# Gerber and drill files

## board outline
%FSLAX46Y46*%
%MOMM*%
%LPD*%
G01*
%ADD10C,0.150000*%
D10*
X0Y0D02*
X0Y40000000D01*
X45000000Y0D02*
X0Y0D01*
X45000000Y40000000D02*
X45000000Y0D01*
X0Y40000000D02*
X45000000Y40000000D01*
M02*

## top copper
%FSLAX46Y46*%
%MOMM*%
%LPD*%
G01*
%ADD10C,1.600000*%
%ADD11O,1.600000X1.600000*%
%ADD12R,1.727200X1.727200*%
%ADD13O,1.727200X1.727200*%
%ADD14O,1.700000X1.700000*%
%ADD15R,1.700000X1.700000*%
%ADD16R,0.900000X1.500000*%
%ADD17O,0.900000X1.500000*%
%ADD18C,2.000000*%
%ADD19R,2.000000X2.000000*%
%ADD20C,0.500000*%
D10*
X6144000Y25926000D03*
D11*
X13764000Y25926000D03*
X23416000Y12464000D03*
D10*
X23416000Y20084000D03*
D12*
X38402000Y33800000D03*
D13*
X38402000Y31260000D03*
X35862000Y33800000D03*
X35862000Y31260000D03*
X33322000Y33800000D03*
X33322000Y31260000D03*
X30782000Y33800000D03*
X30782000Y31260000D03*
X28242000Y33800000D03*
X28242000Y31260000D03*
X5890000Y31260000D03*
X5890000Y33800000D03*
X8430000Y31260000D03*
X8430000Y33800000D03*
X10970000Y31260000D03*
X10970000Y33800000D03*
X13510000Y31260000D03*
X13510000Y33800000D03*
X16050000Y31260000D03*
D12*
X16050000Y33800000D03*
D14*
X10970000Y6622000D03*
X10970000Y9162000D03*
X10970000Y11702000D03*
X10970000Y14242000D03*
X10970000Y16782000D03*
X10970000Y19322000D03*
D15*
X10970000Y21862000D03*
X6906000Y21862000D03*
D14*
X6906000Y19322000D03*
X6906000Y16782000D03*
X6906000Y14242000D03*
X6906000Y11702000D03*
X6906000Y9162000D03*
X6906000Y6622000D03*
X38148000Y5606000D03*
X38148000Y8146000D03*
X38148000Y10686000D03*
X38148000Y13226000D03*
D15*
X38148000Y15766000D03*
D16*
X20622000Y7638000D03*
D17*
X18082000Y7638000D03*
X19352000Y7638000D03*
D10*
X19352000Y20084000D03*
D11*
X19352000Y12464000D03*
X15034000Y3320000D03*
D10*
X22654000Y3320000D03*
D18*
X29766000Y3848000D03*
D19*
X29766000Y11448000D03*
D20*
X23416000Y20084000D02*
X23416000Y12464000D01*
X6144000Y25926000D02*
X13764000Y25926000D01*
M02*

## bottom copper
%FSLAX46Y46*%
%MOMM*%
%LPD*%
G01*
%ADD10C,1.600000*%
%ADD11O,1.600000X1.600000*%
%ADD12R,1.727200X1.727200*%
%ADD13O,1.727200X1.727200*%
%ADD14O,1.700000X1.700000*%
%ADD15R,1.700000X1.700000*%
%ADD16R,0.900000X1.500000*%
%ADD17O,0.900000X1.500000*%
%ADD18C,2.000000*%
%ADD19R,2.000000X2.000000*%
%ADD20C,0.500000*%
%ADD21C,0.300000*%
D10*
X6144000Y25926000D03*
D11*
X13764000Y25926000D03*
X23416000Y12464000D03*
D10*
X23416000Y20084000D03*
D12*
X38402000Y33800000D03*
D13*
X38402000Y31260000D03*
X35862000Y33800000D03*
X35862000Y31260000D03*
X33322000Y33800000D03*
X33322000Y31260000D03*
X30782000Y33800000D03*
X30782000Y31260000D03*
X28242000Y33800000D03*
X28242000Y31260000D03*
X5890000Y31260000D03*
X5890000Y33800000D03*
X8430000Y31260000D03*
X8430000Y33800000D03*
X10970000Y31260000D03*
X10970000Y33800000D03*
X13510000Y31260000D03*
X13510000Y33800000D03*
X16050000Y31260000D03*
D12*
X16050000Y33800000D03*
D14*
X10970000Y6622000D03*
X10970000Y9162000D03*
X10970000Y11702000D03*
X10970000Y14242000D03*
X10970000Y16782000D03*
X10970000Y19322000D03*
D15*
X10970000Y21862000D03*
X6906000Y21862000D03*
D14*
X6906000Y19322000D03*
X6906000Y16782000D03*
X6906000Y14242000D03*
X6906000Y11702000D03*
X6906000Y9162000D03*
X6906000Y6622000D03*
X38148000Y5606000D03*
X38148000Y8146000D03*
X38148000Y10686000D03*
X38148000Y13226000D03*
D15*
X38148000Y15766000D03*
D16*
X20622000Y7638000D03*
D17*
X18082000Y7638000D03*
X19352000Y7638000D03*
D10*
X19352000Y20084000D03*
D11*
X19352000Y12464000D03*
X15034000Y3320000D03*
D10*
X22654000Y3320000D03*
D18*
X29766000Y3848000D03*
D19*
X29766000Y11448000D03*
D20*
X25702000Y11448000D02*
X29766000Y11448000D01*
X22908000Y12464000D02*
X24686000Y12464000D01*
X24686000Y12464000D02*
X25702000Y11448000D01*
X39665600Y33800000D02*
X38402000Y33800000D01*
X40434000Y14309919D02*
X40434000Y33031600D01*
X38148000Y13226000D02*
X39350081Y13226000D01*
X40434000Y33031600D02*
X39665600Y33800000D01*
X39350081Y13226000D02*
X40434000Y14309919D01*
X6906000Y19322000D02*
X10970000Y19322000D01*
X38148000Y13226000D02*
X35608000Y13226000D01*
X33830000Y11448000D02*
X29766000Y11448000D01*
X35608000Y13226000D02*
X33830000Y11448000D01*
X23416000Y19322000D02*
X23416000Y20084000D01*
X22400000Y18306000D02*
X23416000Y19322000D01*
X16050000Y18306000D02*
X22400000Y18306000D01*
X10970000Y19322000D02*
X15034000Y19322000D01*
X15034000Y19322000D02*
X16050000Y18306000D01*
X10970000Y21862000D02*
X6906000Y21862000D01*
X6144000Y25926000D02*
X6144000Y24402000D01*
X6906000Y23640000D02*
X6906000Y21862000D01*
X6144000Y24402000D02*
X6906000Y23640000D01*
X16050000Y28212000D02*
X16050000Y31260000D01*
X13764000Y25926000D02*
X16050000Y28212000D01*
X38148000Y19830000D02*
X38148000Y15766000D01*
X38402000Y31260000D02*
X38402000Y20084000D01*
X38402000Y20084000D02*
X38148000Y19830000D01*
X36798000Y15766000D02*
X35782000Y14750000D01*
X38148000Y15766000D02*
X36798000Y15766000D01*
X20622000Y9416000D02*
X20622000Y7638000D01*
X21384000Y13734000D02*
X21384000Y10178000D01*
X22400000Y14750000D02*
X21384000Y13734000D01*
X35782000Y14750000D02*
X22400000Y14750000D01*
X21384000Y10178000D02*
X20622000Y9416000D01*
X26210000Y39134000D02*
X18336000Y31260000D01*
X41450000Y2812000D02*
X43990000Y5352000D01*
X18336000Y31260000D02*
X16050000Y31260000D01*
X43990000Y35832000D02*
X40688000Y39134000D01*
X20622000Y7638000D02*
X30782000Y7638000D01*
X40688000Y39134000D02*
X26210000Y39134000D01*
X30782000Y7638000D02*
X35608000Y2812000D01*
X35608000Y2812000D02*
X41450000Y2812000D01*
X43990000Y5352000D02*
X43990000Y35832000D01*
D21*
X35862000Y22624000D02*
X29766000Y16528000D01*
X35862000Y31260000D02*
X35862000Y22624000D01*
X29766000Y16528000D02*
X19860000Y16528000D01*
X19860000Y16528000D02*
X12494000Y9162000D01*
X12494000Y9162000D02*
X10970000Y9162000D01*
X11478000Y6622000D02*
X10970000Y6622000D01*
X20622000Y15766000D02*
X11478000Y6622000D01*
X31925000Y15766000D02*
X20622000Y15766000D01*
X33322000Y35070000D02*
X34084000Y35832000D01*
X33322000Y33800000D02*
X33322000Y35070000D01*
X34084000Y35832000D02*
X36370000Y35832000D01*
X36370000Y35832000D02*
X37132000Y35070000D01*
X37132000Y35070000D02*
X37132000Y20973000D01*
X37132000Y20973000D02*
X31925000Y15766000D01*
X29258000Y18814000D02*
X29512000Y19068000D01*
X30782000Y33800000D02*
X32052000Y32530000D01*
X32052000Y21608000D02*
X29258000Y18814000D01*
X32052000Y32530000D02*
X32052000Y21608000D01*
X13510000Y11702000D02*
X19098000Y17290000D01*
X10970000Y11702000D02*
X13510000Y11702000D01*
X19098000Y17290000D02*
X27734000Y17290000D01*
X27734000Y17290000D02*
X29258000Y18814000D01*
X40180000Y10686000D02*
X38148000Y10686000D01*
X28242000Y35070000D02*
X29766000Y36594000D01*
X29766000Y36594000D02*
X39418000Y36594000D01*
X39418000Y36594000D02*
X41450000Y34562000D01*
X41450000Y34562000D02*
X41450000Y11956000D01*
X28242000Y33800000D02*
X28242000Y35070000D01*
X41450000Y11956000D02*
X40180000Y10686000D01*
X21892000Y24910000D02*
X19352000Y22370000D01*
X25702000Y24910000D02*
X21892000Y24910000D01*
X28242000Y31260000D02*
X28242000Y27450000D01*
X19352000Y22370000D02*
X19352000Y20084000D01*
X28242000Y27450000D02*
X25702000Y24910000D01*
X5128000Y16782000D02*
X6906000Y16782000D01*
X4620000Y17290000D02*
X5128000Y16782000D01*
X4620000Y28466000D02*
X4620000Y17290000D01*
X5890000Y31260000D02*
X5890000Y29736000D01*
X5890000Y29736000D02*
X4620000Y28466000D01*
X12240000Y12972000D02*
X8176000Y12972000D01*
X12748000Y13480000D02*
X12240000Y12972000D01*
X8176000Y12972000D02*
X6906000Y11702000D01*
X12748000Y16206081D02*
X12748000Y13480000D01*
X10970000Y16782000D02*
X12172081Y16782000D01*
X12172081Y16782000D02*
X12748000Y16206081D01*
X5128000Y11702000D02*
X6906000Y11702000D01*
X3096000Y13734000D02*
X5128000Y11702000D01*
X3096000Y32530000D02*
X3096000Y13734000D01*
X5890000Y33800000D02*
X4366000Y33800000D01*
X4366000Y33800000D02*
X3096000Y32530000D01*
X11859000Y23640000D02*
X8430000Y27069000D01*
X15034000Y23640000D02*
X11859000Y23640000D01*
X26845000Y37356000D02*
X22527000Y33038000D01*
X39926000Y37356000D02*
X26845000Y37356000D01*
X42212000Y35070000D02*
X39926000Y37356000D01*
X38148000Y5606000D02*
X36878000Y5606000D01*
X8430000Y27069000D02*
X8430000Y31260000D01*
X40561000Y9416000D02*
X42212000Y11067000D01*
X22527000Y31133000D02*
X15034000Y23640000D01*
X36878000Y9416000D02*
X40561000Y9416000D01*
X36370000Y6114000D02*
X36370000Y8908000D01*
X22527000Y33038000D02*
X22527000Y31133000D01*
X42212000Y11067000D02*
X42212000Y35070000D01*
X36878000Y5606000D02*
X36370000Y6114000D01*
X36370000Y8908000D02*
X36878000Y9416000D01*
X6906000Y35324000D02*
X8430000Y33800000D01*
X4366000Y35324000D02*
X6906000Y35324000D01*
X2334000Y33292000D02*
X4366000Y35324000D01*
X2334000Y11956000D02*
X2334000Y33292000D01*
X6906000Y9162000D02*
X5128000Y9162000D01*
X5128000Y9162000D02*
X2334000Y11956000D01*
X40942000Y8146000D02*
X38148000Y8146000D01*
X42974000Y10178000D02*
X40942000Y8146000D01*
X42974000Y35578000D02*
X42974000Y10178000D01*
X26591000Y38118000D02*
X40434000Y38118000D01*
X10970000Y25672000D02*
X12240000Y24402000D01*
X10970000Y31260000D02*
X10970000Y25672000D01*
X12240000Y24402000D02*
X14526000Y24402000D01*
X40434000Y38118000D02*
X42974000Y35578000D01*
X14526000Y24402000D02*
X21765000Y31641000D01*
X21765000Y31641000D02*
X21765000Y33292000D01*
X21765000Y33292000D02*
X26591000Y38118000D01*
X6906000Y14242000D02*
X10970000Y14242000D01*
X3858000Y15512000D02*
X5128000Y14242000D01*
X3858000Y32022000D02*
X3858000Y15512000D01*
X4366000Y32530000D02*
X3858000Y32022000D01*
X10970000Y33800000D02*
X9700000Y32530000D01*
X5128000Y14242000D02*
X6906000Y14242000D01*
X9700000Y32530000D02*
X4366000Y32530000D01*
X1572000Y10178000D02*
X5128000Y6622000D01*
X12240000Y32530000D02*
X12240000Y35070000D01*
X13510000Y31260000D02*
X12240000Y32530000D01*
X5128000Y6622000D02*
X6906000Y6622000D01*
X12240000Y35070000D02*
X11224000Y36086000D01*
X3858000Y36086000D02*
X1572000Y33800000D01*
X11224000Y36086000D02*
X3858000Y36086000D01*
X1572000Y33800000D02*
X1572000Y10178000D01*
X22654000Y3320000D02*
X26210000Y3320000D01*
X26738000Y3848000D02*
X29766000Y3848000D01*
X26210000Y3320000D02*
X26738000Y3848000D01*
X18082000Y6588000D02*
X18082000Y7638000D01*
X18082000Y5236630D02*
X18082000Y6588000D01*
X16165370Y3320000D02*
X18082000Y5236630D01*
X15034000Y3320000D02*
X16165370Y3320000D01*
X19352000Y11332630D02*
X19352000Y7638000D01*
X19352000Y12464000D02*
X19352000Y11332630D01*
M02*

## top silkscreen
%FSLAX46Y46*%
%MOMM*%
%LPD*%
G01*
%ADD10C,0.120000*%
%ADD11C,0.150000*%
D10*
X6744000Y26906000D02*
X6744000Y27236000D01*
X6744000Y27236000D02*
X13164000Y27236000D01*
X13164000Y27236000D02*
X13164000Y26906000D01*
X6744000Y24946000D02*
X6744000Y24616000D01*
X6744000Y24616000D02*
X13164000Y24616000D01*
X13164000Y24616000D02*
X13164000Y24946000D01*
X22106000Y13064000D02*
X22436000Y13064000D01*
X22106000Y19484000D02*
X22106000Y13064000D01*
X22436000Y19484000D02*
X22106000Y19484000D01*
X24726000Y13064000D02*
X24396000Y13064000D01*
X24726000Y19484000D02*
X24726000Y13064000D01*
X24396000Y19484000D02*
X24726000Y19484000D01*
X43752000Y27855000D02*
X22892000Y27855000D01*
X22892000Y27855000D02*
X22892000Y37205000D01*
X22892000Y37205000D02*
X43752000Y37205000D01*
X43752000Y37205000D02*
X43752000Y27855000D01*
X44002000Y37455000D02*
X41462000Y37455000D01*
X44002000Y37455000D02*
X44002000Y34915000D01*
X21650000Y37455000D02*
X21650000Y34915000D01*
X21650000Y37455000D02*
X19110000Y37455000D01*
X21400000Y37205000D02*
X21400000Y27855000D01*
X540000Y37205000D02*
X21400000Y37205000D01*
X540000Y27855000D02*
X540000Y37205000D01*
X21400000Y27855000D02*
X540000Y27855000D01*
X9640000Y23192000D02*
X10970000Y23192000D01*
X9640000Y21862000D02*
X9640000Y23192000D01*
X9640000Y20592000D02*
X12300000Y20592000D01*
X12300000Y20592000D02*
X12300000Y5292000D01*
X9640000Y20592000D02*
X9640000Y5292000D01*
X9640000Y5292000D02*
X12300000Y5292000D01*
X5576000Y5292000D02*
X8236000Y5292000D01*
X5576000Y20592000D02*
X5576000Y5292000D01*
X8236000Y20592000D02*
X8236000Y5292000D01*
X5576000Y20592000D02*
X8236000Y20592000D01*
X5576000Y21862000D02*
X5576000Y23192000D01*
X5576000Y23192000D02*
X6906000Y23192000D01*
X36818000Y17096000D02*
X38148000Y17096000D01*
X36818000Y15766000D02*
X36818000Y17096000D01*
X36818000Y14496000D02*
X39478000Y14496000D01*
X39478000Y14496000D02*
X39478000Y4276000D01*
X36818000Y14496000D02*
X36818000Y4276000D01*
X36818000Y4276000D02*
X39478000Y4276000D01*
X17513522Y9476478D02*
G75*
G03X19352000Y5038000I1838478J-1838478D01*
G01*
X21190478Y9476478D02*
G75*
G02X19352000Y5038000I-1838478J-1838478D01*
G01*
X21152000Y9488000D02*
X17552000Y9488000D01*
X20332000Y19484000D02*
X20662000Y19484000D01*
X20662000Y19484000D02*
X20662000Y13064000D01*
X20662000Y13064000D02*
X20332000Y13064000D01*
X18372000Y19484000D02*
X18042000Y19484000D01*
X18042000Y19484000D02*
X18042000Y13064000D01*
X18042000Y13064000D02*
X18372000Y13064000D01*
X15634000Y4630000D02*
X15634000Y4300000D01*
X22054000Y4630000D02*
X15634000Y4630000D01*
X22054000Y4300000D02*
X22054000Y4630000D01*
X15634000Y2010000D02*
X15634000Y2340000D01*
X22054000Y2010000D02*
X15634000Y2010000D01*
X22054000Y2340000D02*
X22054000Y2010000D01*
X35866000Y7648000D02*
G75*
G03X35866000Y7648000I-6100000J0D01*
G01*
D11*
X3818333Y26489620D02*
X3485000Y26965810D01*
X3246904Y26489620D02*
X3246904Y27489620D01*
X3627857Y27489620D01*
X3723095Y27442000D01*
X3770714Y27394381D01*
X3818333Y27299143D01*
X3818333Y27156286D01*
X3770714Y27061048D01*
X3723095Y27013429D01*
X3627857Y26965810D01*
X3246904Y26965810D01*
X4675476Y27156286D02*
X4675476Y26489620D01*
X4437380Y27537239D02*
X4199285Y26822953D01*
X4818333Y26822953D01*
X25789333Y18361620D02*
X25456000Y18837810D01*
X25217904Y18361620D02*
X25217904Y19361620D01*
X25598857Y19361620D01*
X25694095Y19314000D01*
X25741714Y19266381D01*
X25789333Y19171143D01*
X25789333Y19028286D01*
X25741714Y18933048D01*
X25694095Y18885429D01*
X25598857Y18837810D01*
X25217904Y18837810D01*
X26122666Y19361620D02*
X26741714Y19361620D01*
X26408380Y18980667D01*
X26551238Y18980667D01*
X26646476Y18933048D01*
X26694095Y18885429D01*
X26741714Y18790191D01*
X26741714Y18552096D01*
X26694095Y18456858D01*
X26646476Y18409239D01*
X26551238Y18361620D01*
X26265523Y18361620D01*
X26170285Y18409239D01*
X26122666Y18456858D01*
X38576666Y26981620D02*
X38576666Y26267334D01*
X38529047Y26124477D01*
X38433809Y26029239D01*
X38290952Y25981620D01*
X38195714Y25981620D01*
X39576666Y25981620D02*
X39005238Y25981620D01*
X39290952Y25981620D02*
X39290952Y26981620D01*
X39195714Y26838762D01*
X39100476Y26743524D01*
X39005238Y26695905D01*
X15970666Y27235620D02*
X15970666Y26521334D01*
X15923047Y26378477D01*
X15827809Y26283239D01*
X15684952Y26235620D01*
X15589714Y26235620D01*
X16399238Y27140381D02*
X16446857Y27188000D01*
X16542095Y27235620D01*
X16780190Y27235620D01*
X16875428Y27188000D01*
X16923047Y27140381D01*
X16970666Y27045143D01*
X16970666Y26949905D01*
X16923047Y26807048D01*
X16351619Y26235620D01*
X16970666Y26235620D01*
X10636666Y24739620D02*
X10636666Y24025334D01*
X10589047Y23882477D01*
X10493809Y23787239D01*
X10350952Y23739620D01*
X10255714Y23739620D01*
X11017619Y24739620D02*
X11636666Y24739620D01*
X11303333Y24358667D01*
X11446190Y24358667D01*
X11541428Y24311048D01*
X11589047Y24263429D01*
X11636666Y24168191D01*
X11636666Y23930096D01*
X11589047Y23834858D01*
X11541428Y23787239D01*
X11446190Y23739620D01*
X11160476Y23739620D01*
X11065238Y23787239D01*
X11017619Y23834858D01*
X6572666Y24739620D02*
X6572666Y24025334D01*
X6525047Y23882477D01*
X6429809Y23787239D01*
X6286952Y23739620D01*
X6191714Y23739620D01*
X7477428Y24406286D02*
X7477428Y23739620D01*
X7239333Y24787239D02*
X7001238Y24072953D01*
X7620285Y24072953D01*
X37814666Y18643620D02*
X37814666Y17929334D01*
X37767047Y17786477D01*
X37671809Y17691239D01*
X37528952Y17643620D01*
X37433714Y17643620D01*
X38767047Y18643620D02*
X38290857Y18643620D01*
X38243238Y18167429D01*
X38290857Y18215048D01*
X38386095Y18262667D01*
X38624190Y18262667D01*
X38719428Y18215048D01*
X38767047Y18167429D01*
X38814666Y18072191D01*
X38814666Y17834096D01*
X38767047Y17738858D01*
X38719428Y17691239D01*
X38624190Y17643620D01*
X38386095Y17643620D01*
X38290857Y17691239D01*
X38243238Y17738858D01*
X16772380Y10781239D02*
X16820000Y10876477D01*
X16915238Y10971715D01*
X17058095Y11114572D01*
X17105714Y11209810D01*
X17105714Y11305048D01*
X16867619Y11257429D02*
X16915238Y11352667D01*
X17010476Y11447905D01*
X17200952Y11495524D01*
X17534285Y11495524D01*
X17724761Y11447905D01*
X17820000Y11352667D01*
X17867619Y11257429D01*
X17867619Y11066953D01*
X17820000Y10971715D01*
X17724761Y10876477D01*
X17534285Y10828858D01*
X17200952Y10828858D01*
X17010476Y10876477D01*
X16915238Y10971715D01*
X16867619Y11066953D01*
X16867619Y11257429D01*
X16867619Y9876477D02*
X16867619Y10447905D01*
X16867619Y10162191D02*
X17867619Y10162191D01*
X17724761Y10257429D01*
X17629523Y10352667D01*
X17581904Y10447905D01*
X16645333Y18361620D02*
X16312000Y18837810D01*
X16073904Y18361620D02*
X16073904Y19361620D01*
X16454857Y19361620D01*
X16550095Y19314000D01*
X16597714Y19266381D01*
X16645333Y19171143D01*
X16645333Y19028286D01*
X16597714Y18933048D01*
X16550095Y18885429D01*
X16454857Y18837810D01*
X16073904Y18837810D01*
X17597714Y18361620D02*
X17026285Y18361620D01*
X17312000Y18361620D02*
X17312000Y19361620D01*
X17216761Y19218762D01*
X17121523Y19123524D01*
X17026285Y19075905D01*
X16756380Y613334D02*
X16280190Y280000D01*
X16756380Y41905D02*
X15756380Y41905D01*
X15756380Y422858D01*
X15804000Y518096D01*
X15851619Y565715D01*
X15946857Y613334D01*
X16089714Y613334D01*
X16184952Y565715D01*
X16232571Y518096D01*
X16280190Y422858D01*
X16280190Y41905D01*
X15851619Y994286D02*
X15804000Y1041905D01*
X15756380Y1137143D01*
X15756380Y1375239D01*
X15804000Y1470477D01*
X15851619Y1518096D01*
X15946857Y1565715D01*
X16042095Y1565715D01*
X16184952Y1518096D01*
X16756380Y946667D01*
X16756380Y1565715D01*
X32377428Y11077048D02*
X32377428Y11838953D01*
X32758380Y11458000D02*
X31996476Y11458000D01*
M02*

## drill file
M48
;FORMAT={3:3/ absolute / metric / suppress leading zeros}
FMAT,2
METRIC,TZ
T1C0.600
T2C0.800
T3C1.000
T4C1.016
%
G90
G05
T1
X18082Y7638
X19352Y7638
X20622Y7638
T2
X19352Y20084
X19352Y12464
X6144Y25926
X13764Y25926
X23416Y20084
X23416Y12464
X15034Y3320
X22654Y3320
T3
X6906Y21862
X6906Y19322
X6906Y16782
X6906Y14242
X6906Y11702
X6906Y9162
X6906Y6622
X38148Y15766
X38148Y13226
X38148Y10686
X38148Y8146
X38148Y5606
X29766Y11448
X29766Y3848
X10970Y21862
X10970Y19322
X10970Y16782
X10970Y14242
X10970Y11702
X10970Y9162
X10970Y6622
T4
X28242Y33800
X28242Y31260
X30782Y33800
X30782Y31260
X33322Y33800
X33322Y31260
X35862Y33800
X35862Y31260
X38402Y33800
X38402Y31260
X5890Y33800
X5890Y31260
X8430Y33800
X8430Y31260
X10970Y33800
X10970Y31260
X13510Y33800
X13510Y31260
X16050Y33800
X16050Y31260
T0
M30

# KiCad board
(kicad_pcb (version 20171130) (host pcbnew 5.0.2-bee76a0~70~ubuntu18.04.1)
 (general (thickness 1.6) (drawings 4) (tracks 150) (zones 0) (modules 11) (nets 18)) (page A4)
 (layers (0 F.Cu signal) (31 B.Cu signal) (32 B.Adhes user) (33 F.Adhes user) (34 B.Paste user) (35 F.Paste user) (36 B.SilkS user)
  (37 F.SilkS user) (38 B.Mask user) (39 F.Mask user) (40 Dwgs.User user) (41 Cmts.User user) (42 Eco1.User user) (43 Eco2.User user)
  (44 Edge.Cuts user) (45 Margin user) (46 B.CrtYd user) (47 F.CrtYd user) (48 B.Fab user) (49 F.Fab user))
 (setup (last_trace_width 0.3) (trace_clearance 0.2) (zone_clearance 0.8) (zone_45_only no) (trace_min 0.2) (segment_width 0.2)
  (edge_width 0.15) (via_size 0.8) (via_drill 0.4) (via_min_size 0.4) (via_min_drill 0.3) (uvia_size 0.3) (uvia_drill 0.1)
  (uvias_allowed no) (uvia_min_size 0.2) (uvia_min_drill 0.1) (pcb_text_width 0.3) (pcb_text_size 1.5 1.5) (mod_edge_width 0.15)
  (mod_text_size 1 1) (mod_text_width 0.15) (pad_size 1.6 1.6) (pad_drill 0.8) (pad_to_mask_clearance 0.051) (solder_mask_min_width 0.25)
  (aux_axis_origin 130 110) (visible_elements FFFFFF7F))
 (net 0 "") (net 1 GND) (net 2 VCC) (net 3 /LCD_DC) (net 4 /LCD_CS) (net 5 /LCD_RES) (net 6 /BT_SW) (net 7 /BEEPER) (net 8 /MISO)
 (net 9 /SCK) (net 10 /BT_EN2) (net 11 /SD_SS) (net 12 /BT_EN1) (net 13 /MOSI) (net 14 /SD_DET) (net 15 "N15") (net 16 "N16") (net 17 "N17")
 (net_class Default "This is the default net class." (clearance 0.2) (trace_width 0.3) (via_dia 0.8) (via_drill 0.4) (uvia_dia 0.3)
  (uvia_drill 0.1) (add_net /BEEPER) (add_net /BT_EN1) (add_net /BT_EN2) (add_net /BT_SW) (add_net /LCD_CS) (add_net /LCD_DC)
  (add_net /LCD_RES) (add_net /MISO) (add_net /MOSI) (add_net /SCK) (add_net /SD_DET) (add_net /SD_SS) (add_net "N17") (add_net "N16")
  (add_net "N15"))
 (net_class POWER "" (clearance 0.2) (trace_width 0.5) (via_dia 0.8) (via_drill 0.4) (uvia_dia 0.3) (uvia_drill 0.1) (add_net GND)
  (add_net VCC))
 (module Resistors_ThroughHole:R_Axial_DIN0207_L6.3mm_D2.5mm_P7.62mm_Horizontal (layer F.Cu) (at 136.144 84.074)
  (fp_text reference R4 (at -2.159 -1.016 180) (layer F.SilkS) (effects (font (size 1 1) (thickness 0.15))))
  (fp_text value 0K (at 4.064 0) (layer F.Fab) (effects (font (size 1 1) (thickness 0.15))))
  (fp_line (start 0.6 -0.98) (end 0.6 -1.31) (layer F.SilkS) (width 0.12))
  (fp_line (start 0.6 -1.31) (end 7.02 -1.31) (layer F.SilkS) (width 0.12))
  (fp_line (start 7.02 -1.31) (end 7.02 -0.98) (layer F.SilkS) (width 0.12))
  (fp_line (start 0.6 0.98) (end 0.6 1.31) (layer F.SilkS) (width 0.12))
  (fp_line (start 0.6 1.31) (end 7.02 1.31) (layer F.SilkS) (width 0.12))
  (fp_line (start 7.02 1.31) (end 7.02 0.98) (layer F.SilkS) (width 0.12))
  (pad 1 thru_hole circle (at 0 0) (size 1.6 1.6) (drill 0.8) (layers *.Cu *.Mask) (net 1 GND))
  (pad 2 thru_hole oval (at 7.62 0) (size 1.6 1.6) (drill 0.8) (layers *.Cu *.Mask) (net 1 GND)))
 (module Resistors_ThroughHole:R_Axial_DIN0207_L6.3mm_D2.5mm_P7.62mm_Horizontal (layer F.Cu) (at 153.416 89.916 270)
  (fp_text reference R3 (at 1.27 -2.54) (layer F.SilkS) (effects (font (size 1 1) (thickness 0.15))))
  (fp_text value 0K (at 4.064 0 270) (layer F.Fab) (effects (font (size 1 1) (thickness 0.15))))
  (fp_line (start 7.02 1.31) (end 7.02 0.98) (layer F.SilkS) (width 0.12))
  (fp_line (start 0.6 1.31) (end 7.02 1.31) (layer F.SilkS) (width 0.12))
  (fp_line (start 0.6 0.98) (end 0.6 1.31) (layer F.SilkS) (width 0.12))
  (fp_line (start 7.02 -1.31) (end 7.02 -0.98) (layer F.SilkS) (width 0.12))
  (fp_line (start 0.6 -1.31) (end 7.02 -1.31) (layer F.SilkS) (width 0.12))
  (fp_line (start 0.6 -0.98) (end 0.6 -1.31) (layer F.SilkS) (width 0.12))
  (pad 2 thru_hole oval (at 7.62 0 270) (size 1.6 1.6) (drill 0.8) (layers *.Cu *.Mask) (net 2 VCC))
  (pad 1 thru_hole circle (at 0 0 270) (size 1.6 1.6) (drill 0.8) (layers *.Cu *.Mask) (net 2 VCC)))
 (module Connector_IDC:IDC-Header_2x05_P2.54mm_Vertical (layer F.Cu) (at 168.402 76.2 270)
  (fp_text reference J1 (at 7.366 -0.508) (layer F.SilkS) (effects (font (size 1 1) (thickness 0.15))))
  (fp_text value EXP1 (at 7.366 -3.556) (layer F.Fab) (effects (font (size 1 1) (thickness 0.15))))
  (fp_line (start 5.945 -5.35) (end 5.945 15.51) (layer F.SilkS) (width 0.12))
  (fp_line (start 5.945 15.51) (end -3.405 15.51) (layer F.SilkS) (width 0.12))
  (fp_line (start -3.405 15.51) (end -3.405 -5.35) (layer F.SilkS) (width 0.12))
  (fp_line (start -3.405 -5.35) (end 5.945 -5.35) (layer F.SilkS) (width 0.12))
  (fp_line (start -3.655 -5.6) (end -3.655 -3.06) (layer F.SilkS) (width 0.12))
  (fp_line (start -3.655 -5.6) (end -1.115 -5.6) (layer F.SilkS) (width 0.12))
  (pad 1 thru_hole rect (at 0 0 270) (size 1.7272 1.7272) (drill 1.016) (layers *.Cu *.Mask) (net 2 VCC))
  (pad 2 thru_hole oval (at 2.54 0 270) (size 1.7272 1.7272) (drill 1.016) (layers *.Cu *.Mask) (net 1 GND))
  (pad 3 thru_hole oval (at 0 2.54 270) (size 1.7272 1.7272) (drill 1.016) (layers *.Cu *.Mask))
  (pad 4 thru_hole oval (at 2.54 2.54 270) (size 1.7272 1.7272) (drill 1.016) (layers *.Cu *.Mask) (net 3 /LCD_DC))
  (pad 5 thru_hole oval (at 0 5.08 270) (size 1.7272 1.7272) (drill 1.016) (layers *.Cu *.Mask) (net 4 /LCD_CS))
  (pad 6 thru_hole oval (at 2.54 5.08 270) (size 1.7272 1.7272) (drill 1.016) (layers *.Cu *.Mask))
  (pad 7 thru_hole oval (at 0 7.62 270) (size 1.7272 1.7272) (drill 1.016) (layers *.Cu *.Mask) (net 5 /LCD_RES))
  (pad 8 thru_hole oval (at 2.54 7.62 270) (size 1.7272 1.7272) (drill 1.016) (layers *.Cu *.Mask))
  (pad 9 thru_hole oval (at 0 10.16 270) (size 1.7272 1.7272) (drill 1.016) (layers *.Cu *.Mask) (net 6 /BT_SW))
  (pad 10 thru_hole oval (at 2.54 10.16 270) (size 1.7272 1.7272) (drill 1.016) (layers *.Cu *.Mask) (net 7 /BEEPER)))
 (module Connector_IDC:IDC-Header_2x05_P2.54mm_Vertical (layer F.Cu) (at 146.05 76.2 270)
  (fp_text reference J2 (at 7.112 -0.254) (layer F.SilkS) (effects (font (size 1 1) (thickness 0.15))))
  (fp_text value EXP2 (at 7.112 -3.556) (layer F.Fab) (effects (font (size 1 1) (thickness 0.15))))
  (fp_line (start -3.655 -5.6) (end -1.115 -5.6) (layer F.SilkS) (width 0.12))
  (fp_line (start -3.655 -5.6) (end -3.655 -3.06) (layer F.SilkS) (width 0.12))
  (fp_line (start -3.405 -5.35) (end 5.945 -5.35) (layer F.SilkS) (width 0.12))
  (fp_line (start -3.405 15.51) (end -3.405 -5.35) (layer F.SilkS) (width 0.12))
  (fp_line (start 5.945 15.51) (end -3.405 15.51) (layer F.SilkS) (width 0.12))
  (fp_line (start 5.945 -5.35) (end 5.945 15.51) (layer F.SilkS) (width 0.12))
  (pad 10 thru_hole oval (at 2.54 10.16 270) (size 1.7272 1.7272) (drill 1.016) (layers *.Cu *.Mask) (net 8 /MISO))
  (pad 9 thru_hole oval (at 0 10.16 270) (size 1.7272 1.7272) (drill 1.016) (layers *.Cu *.Mask) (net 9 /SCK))
  (pad 8 thru_hole oval (at 2.54 7.62 270) (size 1.7272 1.7272) (drill 1.016) (layers *.Cu *.Mask) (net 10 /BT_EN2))
  (pad 7 thru_hole oval (at 0 7.62 270) (size 1.7272 1.7272) (drill 1.016) (layers *.Cu *.Mask) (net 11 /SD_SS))
  (pad 6 thru_hole oval (at 2.54 5.08 270) (size 1.7272 1.7272) (drill 1.016) (layers *.Cu *.Mask) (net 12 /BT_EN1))
  (pad 5 thru_hole oval (at 0 5.08 270) (size 1.7272 1.7272) (drill 1.016) (layers *.Cu *.Mask) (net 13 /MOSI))
  (pad 4 thru_hole oval (at 2.54 2.54 270) (size 1.7272 1.7272) (drill 1.016) (layers *.Cu *.Mask) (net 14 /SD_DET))
  (pad 3 thru_hole oval (at 0 2.54 270) (size 1.7272 1.7272) (drill 1.016) (layers *.Cu *.Mask))
  (pad 2 thru_hole oval (at 2.54 0 270) (size 1.7272 1.7272) (drill 1.016) (layers *.Cu *.Mask) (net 1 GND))
  (pad 1 thru_hole rect (at 0 0 270) (size 1.7272 1.7272) (drill 1.016) (layers *.Cu *.Mask)))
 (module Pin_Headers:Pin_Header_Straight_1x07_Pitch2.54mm (layer F.Cu) (at 140.97 88.138)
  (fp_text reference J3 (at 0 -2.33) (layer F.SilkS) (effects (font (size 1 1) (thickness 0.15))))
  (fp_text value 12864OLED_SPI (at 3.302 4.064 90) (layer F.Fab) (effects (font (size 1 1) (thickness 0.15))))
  (fp_line (start -1.33 -1.33) (end 0 -1.33) (layer F.SilkS) (width 0.12))
  (fp_line (start -1.33 0) (end -1.33 -1.33) (layer F.SilkS) (width 0.12))
  (fp_line (start -1.33 1.27) (end 1.33 1.27) (layer F.SilkS) (width 0.12))
  (fp_line (start 1.33 1.27) (end 1.33 16.57) (layer F.SilkS) (width 0.12))
  (fp_line (start -1.33 1.27) (end -1.33 16.57) (layer F.SilkS) (width 0.12))
  (fp_line (start -1.33 16.57) (end 1.33 16.57) (layer F.SilkS) (width 0.12))
  (pad 7 thru_hole oval (at 0 15.24) (size 1.7 1.7) (drill 1) (layers *.Cu *.Mask) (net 4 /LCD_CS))
  (pad 6 thru_hole oval (at 0 12.7) (size 1.7 1.7) (drill 1) (layers *.Cu *.Mask) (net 3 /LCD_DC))
  (pad 5 thru_hole oval (at 0 10.16) (size 1.7 1.7) (drill 1) (layers *.Cu *.Mask) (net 5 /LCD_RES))
  (pad 4 thru_hole oval (at 0 7.62) (size 1.7 1.7) (drill 1) (layers *.Cu *.Mask) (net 13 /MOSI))
  (pad 3 thru_hole oval (at 0 5.08) (size 1.7 1.7) (drill 1) (layers *.Cu *.Mask) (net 9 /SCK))
  (pad 2 thru_hole oval (at 0 2.54) (size 1.7 1.7) (drill 1) (layers *.Cu *.Mask) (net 2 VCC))
  (pad 1 thru_hole rect (at 0 0) (size 1.7 1.7) (drill 1) (layers *.Cu *.Mask) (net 1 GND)))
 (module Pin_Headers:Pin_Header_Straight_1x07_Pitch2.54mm (layer F.Cu) (at 136.906 88.138)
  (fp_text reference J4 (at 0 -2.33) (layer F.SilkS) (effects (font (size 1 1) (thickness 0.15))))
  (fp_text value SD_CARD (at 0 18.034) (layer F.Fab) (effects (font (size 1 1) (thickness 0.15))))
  (fp_line (start -1.33 16.57) (end 1.33 16.57) (layer F.SilkS) (width 0.12))
  (fp_line (start -1.33 1.27) (end -1.33 16.57) (layer F.SilkS) (width 0.12))
  (fp_line (start 1.33 1.27) (end 1.33 16.57) (layer F.SilkS) (width 0.12))
  (fp_line (start -1.33 1.27) (end 1.33 1.27) (layer F.SilkS) (width 0.12))
  (fp_line (start -1.33 0) (end -1.33 -1.33) (layer F.SilkS) (width 0.12))
  (fp_line (start -1.33 -1.33) (end 0 -1.33) (layer F.SilkS) (width 0.12))
  (pad 1 thru_hole rect (at 0 0) (size 1.7 1.7) (drill 1) (layers *.Cu *.Mask) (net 1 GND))
  (pad 2 thru_hole oval (at 0 2.54) (size 1.7 1.7) (drill 1) (layers *.Cu *.Mask) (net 2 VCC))
  (pad 3 thru_hole oval (at 0 5.08) (size 1.7 1.7) (drill 1) (layers *.Cu *.Mask) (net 8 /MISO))
  (pad 4 thru_hole oval (at 0 7.62) (size 1.7 1.7) (drill 1) (layers *.Cu *.Mask) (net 13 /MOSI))
  (pad 5 thru_hole oval (at 0 10.16) (size 1.7 1.7) (drill 1) (layers *.Cu *.Mask) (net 9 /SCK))
  (pad 6 thru_hole oval (at 0 12.7) (size 1.7 1.7) (drill 1) (layers *.Cu *.Mask) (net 11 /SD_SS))
  (pad 7 thru_hole oval (at 0 15.24) (size 1.7 1.7) (drill 1) (layers *.Cu *.Mask) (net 14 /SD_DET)))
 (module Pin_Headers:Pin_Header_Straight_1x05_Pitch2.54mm (layer F.Cu) (at 168.148 94.234)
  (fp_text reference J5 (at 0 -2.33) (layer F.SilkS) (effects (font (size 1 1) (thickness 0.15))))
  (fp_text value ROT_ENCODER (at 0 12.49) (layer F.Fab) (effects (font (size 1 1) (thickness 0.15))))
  (fp_line (start -1.33 -1.33) (end 0 -1.33) (layer F.SilkS) (width 0.12))
  (fp_line (start -1.33 0) (end -1.33 -1.33) (layer F.SilkS) (width 0.12))
  (fp_line (start -1.33 1.27) (end 1.33 1.27) (layer F.SilkS) (width 0.12))
  (fp_line (start 1.33 1.27) (end 1.33 11.49) (layer F.SilkS) (width 0.12))
  (fp_line (start -1.33 1.27) (end -1.33 11.49) (layer F.SilkS) (width 0.12))
  (fp_line (start -1.33 11.49) (end 1.33 11.49) (layer F.SilkS) (width 0.12))
  (pad 5 thru_hole oval (at 0 10.16) (size 1.7 1.7) (drill 1) (layers *.Cu *.Mask) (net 10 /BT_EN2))
  (pad 4 thru_hole oval (at 0 7.62) (size 1.7 1.7) (drill 1) (layers *.Cu *.Mask) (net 12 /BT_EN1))
  (pad 3 thru_hole oval (at 0 5.08) (size 1.7 1.7) (drill 1) (layers *.Cu *.Mask) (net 6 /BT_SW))
  (pad 2 thru_hole oval (at 0 2.54) (size 1.7 1.7) (drill 1) (layers *.Cu *.Mask) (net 2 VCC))
  (pad 1 thru_hole rect (at 0 0) (size 1.7 1.7) (drill 1) (layers *.Cu *.Mask) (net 1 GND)))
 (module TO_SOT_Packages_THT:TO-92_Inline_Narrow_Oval (layer F.Cu) (at 150.622 102.362 180)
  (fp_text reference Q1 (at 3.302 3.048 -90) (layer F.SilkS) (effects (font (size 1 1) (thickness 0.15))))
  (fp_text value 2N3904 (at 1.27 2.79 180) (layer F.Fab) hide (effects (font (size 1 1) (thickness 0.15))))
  (fp_arc (start 1.27 0) (end 1.27 -2.6) (angle 135) (layer F.SilkS) (width 0.12))
  (fp_arc (start 1.27 0) (end 1.27 -2.6) (angle -135) (layer F.SilkS) (width 0.12))
  (fp_line (start -0.53 1.85) (end 3.07 1.85) (layer F.SilkS) (width 0.12))
  (pad 1 thru_hole rect (at 0 0) (size 0.9 1.5) (drill 0.6) (layers *.Cu *.Mask) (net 1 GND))
  (pad 3 thru_hole oval (at 2.54 0) (size 0.9 1.5) (drill 0.6) (layers *.Cu *.Mask) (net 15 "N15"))
  (pad 2 thru_hole oval (at 1.27 0) (size 0.9 1.5) (drill 0.6) (layers *.Cu *.Mask) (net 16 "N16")))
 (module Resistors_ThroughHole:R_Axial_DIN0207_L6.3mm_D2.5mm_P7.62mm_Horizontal (layer F.Cu) (at 149.352 89.916 270)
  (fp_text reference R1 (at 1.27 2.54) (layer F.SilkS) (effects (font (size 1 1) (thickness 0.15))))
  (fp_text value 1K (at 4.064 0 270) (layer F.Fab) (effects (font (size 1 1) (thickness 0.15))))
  (fp_line (start 0.6 -0.98) (end 0.6 -1.31) (layer F.SilkS) (width 0.12))
  (fp_line (start 0.6 -1.31) (end 7.02 -1.31) (layer F.SilkS) (width 0.12))
  (fp_line (start 7.02 -1.31) (end 7.02 -0.98) (layer F.SilkS) (width 0.12))
  (fp_line (start 0.6 0.98) (end 0.6 1.31) (layer F.SilkS) (width 0.12))
  (fp_line (start 0.6 1.31) (end 7.02 1.31) (layer F.SilkS) (width 0.12))
  (fp_line (start 7.02 1.31) (end 7.02 0.98) (layer F.SilkS) (width 0.12))
  (pad 1 thru_hole circle (at 0 0 270) (size 1.6 1.6) (drill 0.8) (layers *.Cu *.Mask) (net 7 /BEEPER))
  (pad 2 thru_hole oval (at 7.62 0 270) (size 1.6 1.6) (drill 0.8) (layers *.Cu *.Mask) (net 16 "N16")))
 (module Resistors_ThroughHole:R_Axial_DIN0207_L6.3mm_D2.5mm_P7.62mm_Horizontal (layer F.Cu) (at 152.654 106.68 180)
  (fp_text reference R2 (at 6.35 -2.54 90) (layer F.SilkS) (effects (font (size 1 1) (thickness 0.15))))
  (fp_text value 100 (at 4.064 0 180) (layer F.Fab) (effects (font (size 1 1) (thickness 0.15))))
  (fp_line (start 7.02 1.31) (end 7.02 0.98) (layer F.SilkS) (width 0.12))
  (fp_line (start 0.6 1.31) (end 7.02 1.31) (layer F.SilkS) (width 0.12))
  (fp_line (start 0.6 0.98) (end 0.6 1.31) (layer F.SilkS) (width 0.12))
  (fp_line (start 7.02 -1.31) (end 7.02 -0.98) (layer F.SilkS) (width 0.12))
  (fp_line (start 0.6 -1.31) (end 7.02 -1.31) (layer F.SilkS) (width 0.12))
  (fp_line (start 0.6 -0.98) (end 0.6 -1.31) (layer F.SilkS) (width 0.12))
  (pad 2 thru_hole oval (at 7.62 0 180) (size 1.6 1.6) (drill 0.8) (layers *.Cu *.Mask) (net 15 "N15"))
  (pad 1 thru_hole circle (at 0 0 180) (size 1.6 1.6) (drill 0.8) (layers *.Cu *.Mask) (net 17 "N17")))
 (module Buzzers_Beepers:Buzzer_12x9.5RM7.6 (layer F.Cu) (at 159.766 98.552 270)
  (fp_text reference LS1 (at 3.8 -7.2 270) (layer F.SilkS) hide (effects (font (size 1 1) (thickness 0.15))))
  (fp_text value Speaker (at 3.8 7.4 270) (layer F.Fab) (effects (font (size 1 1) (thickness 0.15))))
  (fp_circle (center 3.8 0) (end 9.9 0) (layer F.SilkS) (width 0.12))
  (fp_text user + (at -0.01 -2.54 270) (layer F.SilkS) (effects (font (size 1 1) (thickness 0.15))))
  (pad 2 thru_hole circle (at 7.6 0 270) (size 2 2) (drill 1) (layers *.Cu *.Mask) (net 17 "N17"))
  (pad 1 thru_hole rect (at 0 0 270) (size 2 2) (drill 1) (layers *.Cu *.Mask) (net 2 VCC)))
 (gr_line (start 130 110) (end 130 70) (layer Edge.Cuts) (width 0.15))
 (gr_line (start 175 110) (end 130 110) (layer Edge.Cuts) (width 0.15))
 (gr_line (start 175 70) (end 175 110) (layer Edge.Cuts) (width 0.15))
 (gr_line (start 130 70) (end 175 70) (layer Edge.Cuts) (width 0.15))
 (segment (start 155.702 98.552) (end 159.766 98.552) (width 0.5) (layer B.Cu) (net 2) (status 20))
 (segment (start 152.908 97.536) (end 154.686 97.536) (width 0.5) (layer B.Cu) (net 2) (status 10))
 (segment (start 154.686 97.536) (end 155.702 98.552) (width 0.5) (layer B.Cu) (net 2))
 (segment (start 153.416 89.916) (end 153.416 97.536) (width 0.5) (layer F.Cu) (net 2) (status 30))
 (segment (start 169.6656 76.2) (end 168.402 76.2) (width 0.5) (layer B.Cu) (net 2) (status 20))
 (segment (start 170.434 95.690081) (end 170.434 76.9684) (width 0.5) (layer B.Cu) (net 2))
 (segment (start 168.148 96.774) (end 169.350081 96.774) (width 0.5) (layer B.Cu) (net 2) (status 10))
 (segment (start 170.434 76.9684) (end 169.6656 76.2) (width 0.5) (layer B.Cu) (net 2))
 (segment (start 169.350081 96.774) (end 170.434 95.690081) (width 0.5) (layer B.Cu) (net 2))
 (segment (start 136.906 90.678) (end 140.97 90.678) (width 0.5) (layer B.Cu) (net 2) (status 30))
 (segment (start 168.148 96.774) (end 165.608 96.774) (width 0.5) (layer B.Cu) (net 2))
 (segment (start 163.83 98.552) (end 159.766 98.552) (width 0.5) (layer B.Cu) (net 2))
 (segment (start 165.608 96.774) (end 163.83 98.552) (width 0.5) (layer B.Cu) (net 2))
 (segment (start 153.416 90.678) (end 153.416 89.916) (width 0.5) (layer B.Cu) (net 2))
 (segment (start 152.4 91.694) (end 153.416 90.678) (width 0.5) (layer B.Cu) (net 2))
 (segment (start 146.05 91.694) (end 152.4 91.694) (width 0.5) (layer B.Cu) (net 2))
 (segment (start 140.97 90.678) (end 145.034 90.678) (width 0.5) (layer B.Cu) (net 2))
 (segment (start 145.034 90.678) (end 146.05 91.694) (width 0.5) (layer B.Cu) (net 2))
 (segment (start 136.144 84.074) (end 143.764 84.074) (width 0.5) (layer F.Cu) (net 1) (status 30))
 (segment (start 140.97 88.138) (end 136.906 88.138) (width 0.5) (layer B.Cu) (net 1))
 (segment (start 136.144 84.074) (end 136.144 85.598) (width 0.5) (layer B.Cu) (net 1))
 (segment (start 136.906 86.36) (end 136.906 88.138) (width 0.5) (layer B.Cu) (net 1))
 (segment (start 136.144 85.598) (end 136.906 86.36) (width 0.5) (layer B.Cu) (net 1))
 (segment (start 146.05 81.788) (end 146.05 78.74) (width 0.5) (layer B.Cu) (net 1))
 (segment (start 143.764 84.074) (end 146.05 81.788) (width 0.5) (layer B.Cu) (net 1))
 (segment (start 168.148 90.17) (end 168.148 94.234) (width 0.5) (layer B.Cu) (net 1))
 (segment (start 168.402 78.74) (end 168.402 89.916) (width 0.5) (layer B.Cu) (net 1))
 (segment (start 168.402 89.916) (end 168.148 90.17) (width 0.5) (layer B.Cu) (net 1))
 (segment (start 166.798 94.234) (end 165.782 95.25) (width 0.5) (layer B.Cu) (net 1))
 (segment (start 168.148 94.234) (end 166.798 94.234) (width 0.5) (layer B.Cu) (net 1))
 (segment (start 150.622 100.584) (end 150.622 102.362) (width 0.5) (layer B.Cu) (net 1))
 (segment (start 151.384 96.266) (end 151.384 99.822) (width 0.5) (layer B.Cu) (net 1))
 (segment (start 152.4 95.25) (end 151.384 96.266) (width 0.5) (layer B.Cu) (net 1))
 (segment (start 165.782 95.25) (end 152.4 95.25) (width 0.5) (layer B.Cu) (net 1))
 (segment (start 151.384 99.822) (end 150.622 100.584) (width 0.5) (layer B.Cu) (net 1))
 (segment (start 156.21 70.866) (end 148.336 78.74) (width 0.5) (layer B.Cu) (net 1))
 (segment (start 171.45 107.188) (end 173.99 104.648) (width 0.5) (layer B.Cu) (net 1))
 (segment (start 148.336 78.74) (end 146.05 78.74) (width 0.5) (layer B.Cu) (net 1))
 (segment (start 173.99 74.168) (end 170.688 70.866) (width 0.5) (layer B.Cu) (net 1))
 (segment (start 150.622 102.362) (end 160.782 102.362) (width 0.5) (layer B.Cu) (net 1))
 (segment (start 170.688 70.866) (end 156.21 70.866) (width 0.5) (layer B.Cu) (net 1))
 (segment (start 160.782 102.362) (end 165.608 107.188) (width 0.5) (layer B.Cu) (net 1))
 (segment (start 165.608 107.188) (end 171.45 107.188) (width 0.5) (layer B.Cu) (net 1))
 (segment (start 173.99 104.648) (end 173.99 74.168) (width 0.5) (layer B.Cu) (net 1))
 (segment (start 165.862 87.376) (end 159.766 93.472) (width 0.3) (layer B.Cu) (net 3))
 (segment (start 165.862 78.74) (end 165.862 87.376) (width 0.3) (layer B.Cu) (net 3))
 (segment (start 159.766 93.472) (end 149.86 93.472) (width 0.3) (layer B.Cu) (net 3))
 (segment (start 149.86 93.472) (end 142.494 100.838) (width 0.3) (layer B.Cu) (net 3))
 (segment (start 142.494 100.838) (end 140.97 100.838) (width 0.3) (layer B.Cu) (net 3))
 (segment (start 141.478 103.378) (end 140.97 103.378) (width 0.3) (layer B.Cu) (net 4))
 (segment (start 150.622 94.234) (end 141.478 103.378) (width 0.3) (layer B.Cu) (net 4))
 (segment (start 161.925 94.234) (end 150.622 94.234) (width 0.3) (layer B.Cu) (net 4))
 (segment (start 163.322 74.93) (end 164.084 74.168) (width 0.3) (layer B.Cu) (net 4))
 (segment (start 163.322 76.2) (end 163.322 74.93) (width 0.3) (layer B.Cu) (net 4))
 (segment (start 164.084 74.168) (end 166.37 74.168) (width 0.3) (layer B.Cu) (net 4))
 (segment (start 166.37 74.168) (end 167.132 74.93) (width 0.3) (layer B.Cu) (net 4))
 (segment (start 167.132 74.93) (end 167.132 89.027) (width 0.3) (layer B.Cu) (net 4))
 (segment (start 167.132 89.027) (end 161.925 94.234) (width 0.3) (layer B.Cu) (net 4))
 (segment (start 159.258 91.186) (end 159.512 90.932) (width 0.3) (layer B.Cu) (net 5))
 (segment (start 160.782 76.2) (end 162.052 77.47) (width 0.3) (layer B.Cu) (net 5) (status 10))
 (segment (start 162.052 88.392) (end 159.258 91.186) (width 0.3) (layer B.Cu) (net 5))
 (segment (start 162.052 77.47) (end 162.052 88.392) (width 0.3) (layer B.Cu) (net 5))
 (segment (start 143.51 98.298) (end 149.098 92.71) (width 0.3) (layer B.Cu) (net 5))
 (segment (start 140.97 98.298) (end 143.51 98.298) (width 0.3) (layer B.Cu) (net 5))
 (segment (start 149.098 92.71) (end 157.734 92.71) (width 0.3) (layer B.Cu) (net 5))
 (segment (start 157.734 92.71) (end 159.258 91.186) (width 0.3) (layer B.Cu) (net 5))
 (segment (start 170.18 99.314) (end 168.148 99.314) (width 0.3) (layer B.Cu) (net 6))
 (segment (start 158.242 74.93) (end 159.766 73.406) (width 0.3) (layer B.Cu) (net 6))
 (segment (start 159.766 73.406) (end 169.418 73.406) (width 0.3) (layer B.Cu) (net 6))
 (segment (start 169.418 73.406) (end 171.45 75.438) (width 0.3) (layer B.Cu) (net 6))
 (segment (start 171.45 75.438) (end 171.45 98.044) (width 0.3) (layer B.Cu) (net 6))
 (segment (start 158.242 76.2) (end 158.242 74.93) (width 0.3) (layer B.Cu) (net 6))
 (segment (start 171.45 98.044) (end 170.18 99.314) (width 0.3) (layer B.Cu) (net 6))
 (segment (start 151.892 85.09) (end 149.352 87.63) (width 0.3) (layer B.Cu) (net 7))
 (segment (start 155.702 85.09) (end 151.892 85.09) (width 0.3) (layer B.Cu) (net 7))
 (segment (start 158.242 78.74) (end 158.242 82.55) (width 0.3) (layer B.Cu) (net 7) (status 10))
 (segment (start 149.352 87.63) (end 149.352 89.916) (width 0.3) (layer B.Cu) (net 7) (status 20))
 (segment (start 158.242 82.55) (end 155.702 85.09) (width 0.3) (layer B.Cu) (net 7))
 (segment (start 135.128 93.218) (end 136.906 93.218) (width 0.3) (layer B.Cu) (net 8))
 (segment (start 134.62 92.71) (end 135.128 93.218) (width 0.3) (layer B.Cu) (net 8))
 (segment (start 134.62 81.534) (end 134.62 92.71) (width 0.3) (layer B.Cu) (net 8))
 (segment (start 135.89 78.74) (end 135.89 80.264) (width 0.3) (layer B.Cu) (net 8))
 (segment (start 135.89 80.264) (end 134.62 81.534) (width 0.3) (layer B.Cu) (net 8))
 (segment (start 142.24 97.028) (end 138.176 97.028) (width 0.3) (layer B.Cu) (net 9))
 (segment (start 142.748 96.52) (end 142.24 97.028) (width 0.3) (layer B.Cu) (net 9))
 (segment (start 138.176 97.028) (end 136.906 98.298) (width 0.3) (layer B.Cu) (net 9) (status 20))
 (segment (start 142.748 93.793919) (end 142.748 96.52) (width 0.3) (layer B.Cu) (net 9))
 (segment (start 140.97 93.218) (end 142.172081 93.218) (width 0.3) (layer B.Cu) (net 9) (status 10))
 (segment (start 142.172081 93.218) (end 142.748 93.793919) (width 0.3) (layer B.Cu) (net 9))
 (segment (start 135.128 98.298) (end 136.906 98.298) (width 0.3) (layer B.Cu) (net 9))
 (segment (start 133.096 96.266) (end 135.128 98.298) (width 0.3) (layer B.Cu) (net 9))
 (segment (start 133.096 77.47) (end 133.096 96.266) (width 0.3) (layer B.Cu) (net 9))
 (segment (start 135.89 76.2) (end 134.366 76.2) (width 0.3) (layer B.Cu) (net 9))
 (segment (start 134.366 76.2) (end 133.096 77.47) (width 0.3) (layer B.Cu) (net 9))
 (segment (start 141.859 86.36) (end 138.43 82.931) (width 0.3) (layer B.Cu) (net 10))
 (segment (start 145.034 86.36) (end 141.859 86.36) (width 0.3) (layer B.Cu) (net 10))
 (segment (start 156.845 72.644) (end 152.527 76.962) (width 0.3) (layer B.Cu) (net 10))
 (segment (start 169.926 72.644) (end 156.845 72.644) (width 0.3) (layer B.Cu) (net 10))
 (segment (start 172.212 74.93) (end 169.926 72.644) (width 0.3) (layer B.Cu) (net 10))
 (segment (start 168.148 104.394) (end 166.878 104.394) (width 0.3) (layer B.Cu) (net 10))
 (segment (start 138.43 82.931) (end 138.43 78.74) (width 0.3) (layer B.Cu) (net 10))
 (segment (start 170.561 100.584) (end 172.212 98.933) (width 0.3) (layer B.Cu) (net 10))
 (segment (start 152.527 78.867) (end 145.034 86.36) (width 0.3) (layer B.Cu) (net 10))
 (segment (start 166.878 100.584) (end 170.561 100.584) (width 0.3) (layer B.Cu) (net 10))
 (segment (start 166.37 103.886) (end 166.37 101.092) (width 0.3) (layer B.Cu) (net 10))
 (segment (start 152.527 76.962) (end 152.527 78.867) (width 0.3) (layer B.Cu) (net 10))
 (segment (start 172.212 98.933) (end 172.212 74.93) (width 0.3) (layer B.Cu) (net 10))
 (segment (start 166.878 104.394) (end 166.37 103.886) (width 0.3) (layer B.Cu) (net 10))
 (segment (start 166.37 101.092) (end 166.878 100.584) (width 0.3) (layer B.Cu) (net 10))
 (segment (start 136.906 74.676) (end 138.43 76.2) (width 0.3) (layer B.Cu) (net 11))
 (segment (start 134.366 74.676) (end 136.906 74.676) (width 0.3) (layer B.Cu) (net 11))
 (segment (start 132.334 76.708) (end 134.366 74.676) (width 0.3) (layer B.Cu) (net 11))
 (segment (start 132.334 98.044) (end 132.334 76.708) (width 0.3) (layer B.Cu) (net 11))
 (segment (start 136.906 100.838) (end 135.128 100.838) (width 0.3) (layer B.Cu) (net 11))
 (segment (start 135.128 100.838) (end 132.334 98.044) (width 0.3) (layer B.Cu) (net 11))
 (segment (start 170.942 101.854) (end 168.148 101.854) (width 0.3) (layer B.Cu) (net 12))
 (segment (start 172.974 99.822) (end 170.942 101.854) (width 0.3) (layer B.Cu) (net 12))
 (segment (start 172.974 74.422) (end 172.974 99.822) (width 0.3) (layer B.Cu) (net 12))
 (segment (start 156.591 71.882) (end 170.434 71.882) (width 0.3) (layer B.Cu) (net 12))
 (segment (start 140.97 84.328) (end 142.24 85.598) (width 0.3) (layer B.Cu) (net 12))
 (segment (start 140.97 78.74) (end 140.97 84.328) (width 0.3) (layer B.Cu) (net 12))
 (segment (start 142.24 85.598) (end 144.526 85.598) (width 0.3) (layer B.Cu) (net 12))
 (segment (start 170.434 71.882) (end 172.974 74.422) (width 0.3) (layer B.Cu) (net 12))
 (segment (start 144.526 85.598) (end 151.765 78.359) (width 0.3) (layer B.Cu) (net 12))
 (segment (start 151.765 78.359) (end 151.765 76.708) (width 0.3) (layer B.Cu) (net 12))
 (segment (start 151.765 76.708) (end 156.591 71.882) (width 0.3) (layer B.Cu) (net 12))
 (segment (start 136.906 95.758) (end 140.97 95.758) (width 0.3) (layer B.Cu) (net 13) (status 30))
 (segment (start 133.858 94.488) (end 135.128 95.758) (width 0.3) (layer B.Cu) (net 13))
 (segment (start 133.858 77.978) (end 133.858 94.488) (width 0.3) (layer B.Cu) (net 13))
 (segment (start 134.366 77.47) (end 133.858 77.978) (width 0.3) (layer B.Cu) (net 13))
 (segment (start 140.97 76.2) (end 139.7 77.47) (width 0.3) (layer B.Cu) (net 13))
 (segment (start 135.128 95.758) (end 136.906 95.758) (width 0.3) (layer B.Cu) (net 13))
 (segment (start 139.7 77.47) (end 134.366 77.47) (width 0.3) (layer B.Cu) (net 13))
 (segment (start 131.572 99.822) (end 135.128 103.378) (width 0.3) (layer B.Cu) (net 14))
 (segment (start 142.24 77.47) (end 142.24 74.93) (width 0.3) (layer B.Cu) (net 14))
 (segment (start 143.51 78.74) (end 142.24 77.47) (width 0.3) (layer B.Cu) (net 14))
 (segment (start 135.128 103.378) (end 136.906 103.378) (width 0.3) (layer B.Cu) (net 14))
 (segment (start 142.24 74.93) (end 141.224 73.914) (width 0.3) (layer B.Cu) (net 14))
 (segment (start 133.858 73.914) (end 131.572 76.2) (width 0.3) (layer B.Cu) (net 14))
 (segment (start 141.224 73.914) (end 133.858 73.914) (width 0.3) (layer B.Cu) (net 14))
 (segment (start 131.572 76.2) (end 131.572 99.822) (width 0.3) (layer B.Cu) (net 14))
 (segment (start 152.654 106.68) (end 156.21 106.68) (width 0.3) (layer B.Cu) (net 17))
 (segment (start 156.738 106.152) (end 159.766 106.152) (width 0.3) (layer B.Cu) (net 17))
 (segment (start 156.21 106.68) (end 156.738 106.152) (width 0.3) (layer B.Cu) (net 17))
 (segment (start 148.082 103.412) (end 148.082 102.362) (width 0.3) (layer B.Cu) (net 15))
 (segment (start 148.082 104.76337) (end 148.082 103.412) (width 0.3) (layer B.Cu) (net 15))
 (segment (start 146.16537 106.68) (end 148.082 104.76337) (width 0.3) (layer B.Cu) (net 15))
 (segment (start 145.034 106.68) (end 146.16537 106.68) (width 0.3) (layer B.Cu) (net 15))
 (segment (start 149.352 98.66737) (end 149.352 102.362) (width 0.3) (layer B.Cu) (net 16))
 (segment (start 149.352 97.536) (end 149.352 98.66737) (width 0.3) (layer B.Cu) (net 16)))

